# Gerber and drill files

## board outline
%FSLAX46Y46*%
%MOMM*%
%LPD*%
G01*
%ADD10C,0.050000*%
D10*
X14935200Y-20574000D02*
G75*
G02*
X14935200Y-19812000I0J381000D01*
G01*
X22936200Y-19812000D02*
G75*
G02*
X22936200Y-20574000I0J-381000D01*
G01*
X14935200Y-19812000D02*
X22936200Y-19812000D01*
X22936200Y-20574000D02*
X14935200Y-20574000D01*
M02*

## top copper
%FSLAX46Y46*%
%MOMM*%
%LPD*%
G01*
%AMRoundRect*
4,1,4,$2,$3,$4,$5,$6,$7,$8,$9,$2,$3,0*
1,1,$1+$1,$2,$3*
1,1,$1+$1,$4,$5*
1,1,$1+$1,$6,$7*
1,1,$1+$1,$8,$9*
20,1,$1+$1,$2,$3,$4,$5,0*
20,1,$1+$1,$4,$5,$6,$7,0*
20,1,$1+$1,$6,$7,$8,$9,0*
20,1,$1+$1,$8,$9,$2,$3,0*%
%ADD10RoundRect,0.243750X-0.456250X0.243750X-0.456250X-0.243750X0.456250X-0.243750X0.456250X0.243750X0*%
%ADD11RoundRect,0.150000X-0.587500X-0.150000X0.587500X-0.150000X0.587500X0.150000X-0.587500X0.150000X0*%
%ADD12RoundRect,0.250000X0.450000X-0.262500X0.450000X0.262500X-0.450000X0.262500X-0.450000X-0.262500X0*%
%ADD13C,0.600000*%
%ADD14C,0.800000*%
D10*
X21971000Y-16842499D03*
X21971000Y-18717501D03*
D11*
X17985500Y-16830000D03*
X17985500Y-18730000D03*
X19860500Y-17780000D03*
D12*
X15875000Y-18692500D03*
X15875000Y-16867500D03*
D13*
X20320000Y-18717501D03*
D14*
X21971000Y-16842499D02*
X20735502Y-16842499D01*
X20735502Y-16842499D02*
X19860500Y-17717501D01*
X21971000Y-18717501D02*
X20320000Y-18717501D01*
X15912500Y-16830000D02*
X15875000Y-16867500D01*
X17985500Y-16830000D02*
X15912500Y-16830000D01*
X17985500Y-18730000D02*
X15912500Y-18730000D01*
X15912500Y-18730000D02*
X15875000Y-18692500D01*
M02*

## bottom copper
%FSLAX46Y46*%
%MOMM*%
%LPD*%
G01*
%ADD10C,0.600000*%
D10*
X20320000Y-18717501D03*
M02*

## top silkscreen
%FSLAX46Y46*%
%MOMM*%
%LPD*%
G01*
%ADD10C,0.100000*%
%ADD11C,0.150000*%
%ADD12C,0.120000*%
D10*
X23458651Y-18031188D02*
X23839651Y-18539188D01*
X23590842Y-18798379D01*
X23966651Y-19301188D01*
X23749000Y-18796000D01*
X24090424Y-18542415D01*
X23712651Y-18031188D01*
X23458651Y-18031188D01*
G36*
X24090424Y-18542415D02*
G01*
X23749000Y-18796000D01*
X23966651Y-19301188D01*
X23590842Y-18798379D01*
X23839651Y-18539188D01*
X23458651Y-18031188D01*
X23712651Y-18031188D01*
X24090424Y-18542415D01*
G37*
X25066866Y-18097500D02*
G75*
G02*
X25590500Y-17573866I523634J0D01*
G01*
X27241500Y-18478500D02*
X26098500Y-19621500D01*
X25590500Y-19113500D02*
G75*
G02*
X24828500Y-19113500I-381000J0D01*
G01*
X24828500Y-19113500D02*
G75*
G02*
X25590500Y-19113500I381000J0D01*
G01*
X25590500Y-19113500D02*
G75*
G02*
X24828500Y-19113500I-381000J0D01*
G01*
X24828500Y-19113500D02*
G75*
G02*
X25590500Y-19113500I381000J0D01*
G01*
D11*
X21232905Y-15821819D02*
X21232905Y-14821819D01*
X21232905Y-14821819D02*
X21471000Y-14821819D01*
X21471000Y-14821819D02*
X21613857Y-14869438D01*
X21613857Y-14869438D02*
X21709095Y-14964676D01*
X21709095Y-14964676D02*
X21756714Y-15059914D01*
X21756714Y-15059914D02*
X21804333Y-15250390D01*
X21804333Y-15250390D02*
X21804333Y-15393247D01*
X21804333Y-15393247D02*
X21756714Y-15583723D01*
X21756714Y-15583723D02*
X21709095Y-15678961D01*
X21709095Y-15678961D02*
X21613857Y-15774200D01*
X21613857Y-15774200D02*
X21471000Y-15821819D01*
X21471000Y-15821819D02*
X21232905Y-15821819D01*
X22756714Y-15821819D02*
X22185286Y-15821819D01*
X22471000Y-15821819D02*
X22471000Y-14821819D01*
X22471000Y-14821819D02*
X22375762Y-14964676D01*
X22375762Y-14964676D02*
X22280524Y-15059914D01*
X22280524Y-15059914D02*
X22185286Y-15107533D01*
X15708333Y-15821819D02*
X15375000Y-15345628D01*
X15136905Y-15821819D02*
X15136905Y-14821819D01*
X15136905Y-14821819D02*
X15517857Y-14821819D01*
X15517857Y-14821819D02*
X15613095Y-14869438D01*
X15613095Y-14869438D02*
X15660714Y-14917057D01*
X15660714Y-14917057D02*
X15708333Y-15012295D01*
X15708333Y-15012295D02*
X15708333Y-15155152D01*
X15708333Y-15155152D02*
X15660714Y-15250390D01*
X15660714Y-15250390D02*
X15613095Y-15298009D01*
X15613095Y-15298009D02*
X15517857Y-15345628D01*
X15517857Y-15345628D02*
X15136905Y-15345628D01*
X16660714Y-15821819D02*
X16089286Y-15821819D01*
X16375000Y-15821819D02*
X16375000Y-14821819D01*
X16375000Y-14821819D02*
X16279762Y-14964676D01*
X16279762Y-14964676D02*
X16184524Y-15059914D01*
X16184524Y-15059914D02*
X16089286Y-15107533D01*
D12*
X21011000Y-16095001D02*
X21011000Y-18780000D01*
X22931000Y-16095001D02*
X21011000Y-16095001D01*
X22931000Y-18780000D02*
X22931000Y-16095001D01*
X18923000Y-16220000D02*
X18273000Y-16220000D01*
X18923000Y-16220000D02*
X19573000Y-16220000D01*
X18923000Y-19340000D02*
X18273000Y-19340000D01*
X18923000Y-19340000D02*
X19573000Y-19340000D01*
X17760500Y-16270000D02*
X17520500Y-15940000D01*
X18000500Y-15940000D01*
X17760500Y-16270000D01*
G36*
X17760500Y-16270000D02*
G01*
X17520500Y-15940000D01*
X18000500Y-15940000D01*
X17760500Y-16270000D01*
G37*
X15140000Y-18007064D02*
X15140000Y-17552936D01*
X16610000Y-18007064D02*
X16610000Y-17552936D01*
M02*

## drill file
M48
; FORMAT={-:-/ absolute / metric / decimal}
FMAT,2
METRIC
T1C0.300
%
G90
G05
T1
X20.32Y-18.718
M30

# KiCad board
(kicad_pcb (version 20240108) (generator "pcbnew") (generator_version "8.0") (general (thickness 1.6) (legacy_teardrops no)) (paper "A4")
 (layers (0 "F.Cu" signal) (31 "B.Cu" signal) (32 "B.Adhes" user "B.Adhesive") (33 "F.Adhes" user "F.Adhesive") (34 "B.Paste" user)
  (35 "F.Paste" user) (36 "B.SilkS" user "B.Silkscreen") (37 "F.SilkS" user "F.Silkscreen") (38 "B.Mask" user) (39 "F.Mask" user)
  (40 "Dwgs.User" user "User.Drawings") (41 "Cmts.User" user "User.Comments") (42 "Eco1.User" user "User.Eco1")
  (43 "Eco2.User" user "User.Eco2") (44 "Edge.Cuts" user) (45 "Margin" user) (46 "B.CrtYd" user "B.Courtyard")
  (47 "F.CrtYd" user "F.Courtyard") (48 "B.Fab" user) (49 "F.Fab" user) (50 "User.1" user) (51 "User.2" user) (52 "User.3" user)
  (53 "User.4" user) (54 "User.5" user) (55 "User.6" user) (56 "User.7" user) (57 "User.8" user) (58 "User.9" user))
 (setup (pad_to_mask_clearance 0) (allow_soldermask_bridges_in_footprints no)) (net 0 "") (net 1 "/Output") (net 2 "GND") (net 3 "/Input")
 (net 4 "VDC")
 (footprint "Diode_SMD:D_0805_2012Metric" (layer "F.Cu") (at 21.971 17.78 -90)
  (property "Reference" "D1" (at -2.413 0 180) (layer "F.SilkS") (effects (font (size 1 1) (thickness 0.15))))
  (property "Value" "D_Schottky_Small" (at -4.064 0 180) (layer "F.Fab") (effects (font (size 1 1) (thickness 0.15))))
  (fp_line (start -1.684999 0.96) (end 1 0.96) (stroke (width 0.12) (type solid)) (layer "F.SilkS"))
  (fp_line (start -1.684999 -0.96) (end -1.684999 0.96) (stroke (width 0.12) (type solid)) (layer "F.SilkS"))
  (fp_line (start 1 -0.96) (end -1.684999 -0.96) (stroke (width 0.12) (type solid)) (layer "F.SilkS"))
  (pad "1" smd roundrect (at -0.937501 0 270) (size 0.975 1.4) (layers "F.Cu" "F.Paste" "F.Mask") (roundrect_rratio 0.25) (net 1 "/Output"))
  (pad "2" smd roundrect (at 0.937501 0 270) (size 0.975 1.4) (layers "F.Cu" "F.Paste" "F.Mask") (roundrect_rratio 0.25) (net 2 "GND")))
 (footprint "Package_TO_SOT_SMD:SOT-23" (layer "F.Cu") (at 18.923 17.78)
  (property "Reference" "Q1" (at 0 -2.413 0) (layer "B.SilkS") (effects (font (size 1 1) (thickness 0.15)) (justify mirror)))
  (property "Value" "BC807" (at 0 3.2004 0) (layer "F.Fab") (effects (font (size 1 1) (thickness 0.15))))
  (fp_line (start 0 -1.56) (end -0.65 -1.56) (stroke (width 0.12) (type solid)) (layer "F.SilkS"))
  (fp_line (start 0 -1.56) (end 0.65 -1.56) (stroke (width 0.12) (type solid)) (layer "F.SilkS"))
  (fp_line (start 0 1.56) (end -0.65 1.56) (stroke (width 0.12) (type solid)) (layer "F.SilkS"))
  (fp_line (start 0 1.56) (end 0.65 1.56) (stroke (width 0.12) (type solid)) (layer "F.SilkS"))
  (fp_poly
   (pts (xy -1.1625 -1.51) (xy -1.4025 -1.84) (xy -0.9225 -1.84) (xy -1.1625 -1.51)) (stroke (width 0.12) (type solid)) (fill solid)
   (layer "F.SilkS"))
  (pad "1" smd roundrect (at -0.9375 -0.95) (size 1.475 0.6) (layers "F.Cu" "F.Paste" "F.Mask") (roundrect_rratio 0.25) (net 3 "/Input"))
  (pad "2" smd roundrect (at -0.9375 0.95) (size 1.475 0.6) (layers "F.Cu" "F.Paste" "F.Mask") (roundrect_rratio 0.25) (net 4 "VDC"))
  (pad "3" smd roundrect (at 0.9375 0) (size 1.475 0.6) (layers "F.Cu" "F.Paste" "F.Mask") (roundrect_rratio 0.25) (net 1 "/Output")))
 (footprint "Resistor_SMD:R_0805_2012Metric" (layer "F.Cu") (at 15.875 17.78 90)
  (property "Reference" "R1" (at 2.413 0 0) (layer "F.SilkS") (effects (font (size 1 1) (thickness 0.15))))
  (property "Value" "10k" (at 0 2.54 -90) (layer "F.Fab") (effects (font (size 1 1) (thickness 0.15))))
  (fp_line (start -0.227064 -0.735) (end 0.227064 -0.735) (stroke (width 0.12) (type solid)) (layer "F.SilkS"))
  (fp_line (start -0.227064 0.735) (end 0.227064 0.735) (stroke (width 0.12) (type solid)) (layer "F.SilkS"))
  (pad "1" smd roundrect (at -0.9125 0 90) (size 1.025 1.4) (layers "F.Cu" "F.Paste" "F.Mask") (roundrect_rratio 0.243902) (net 4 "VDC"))
  (pad "2" smd roundrect (at 0.9125 0 90) (size 1.025 1.4) (layers "F.Cu" "F.Paste" "F.Mask") (roundrect_rratio 0.243902) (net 3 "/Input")))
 (gr_poly
  (pts (xy 23.458651 18.031188) (xy 23.839651 18.539188) (xy 23.590842 18.798379) (xy 23.966651 19.301188) (xy 23.749 18.796)
   (xy 24.090424 18.542415) (xy 23.712651 18.031188))
  (stroke (width 0.1) (type solid)) (fill solid) (layer "F.SilkS"))
 (gr_arc (start 25.066866 18.0975) (mid 25.220235 17.727235) (end 25.5905 17.573866) (stroke (width 0.1) (type default)) (layer "F.SilkS"))
 (gr_line (start 27.2415 18.4785) (end 26.0985 19.6215) (stroke (width 0.1) (type default)) (layer "F.SilkS"))
 (gr_circle (center 25.2095 19.1135) (end 25.2095 18.7325) (stroke (width 0.1) (type default)) (fill none) (layer "F.SilkS"))
 (gr_circle (center 25.2095 19.1135) (end 25.2095 18.7325) (stroke (width 0.1) (type default)) (fill none) (layer "F.SilkS"))
 (gr_arc (start 14.9352 20.574) (mid 14.5542 20.193) (end 14.9352 19.812) (stroke (width 0.05) (type default)) (layer "Edge.Cuts"))
 (gr_arc (start 22.9362 19.812) (mid 23.3172 20.193) (end 22.9362 20.574) (stroke (width 0.05) (type default)) (layer "Edge.Cuts"))
 (gr_line (start 14.9352 19.812) (end 22.9362 19.812) (stroke (width 0.05) (type default)) (layer "Edge.Cuts"))
 (gr_line (start 22.9362 20.574) (end 14.9352 20.574) (stroke (width 0.05) (type default)) (layer "Edge.Cuts"))
 (segment (start 21.971 16.842499) (end 20.735502 16.842499) (width 0.8) (layer "F.Cu") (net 1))
 (segment (start 20.735502 16.842499) (end 19.8605 17.717501) (width 0.8) (layer "F.Cu") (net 1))
 (segment (start 21.971 18.717501) (end 20.32 18.717501) (width 0.8) (layer "F.Cu") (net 2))
 (via (at 20.32 18.717501) (size 0.6) (drill 0.3) (layers "F.Cu" "B.Cu") (free yes) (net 2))
 (segment (start 15.9125 16.83) (end 15.875 16.8675) (width 0.8) (layer "F.Cu") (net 3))
 (segment (start 17.9855 16.83) (end 15.9125 16.83) (width 0.8) (layer "F.Cu") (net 3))
 (segment (start 17.9855 18.73) (end 15.9125 18.73) (width 0.8) (layer "F.Cu") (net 4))
 (segment (start 15.9125 18.73) (end 15.875 18.6925) (width 0.8) (layer "F.Cu") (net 4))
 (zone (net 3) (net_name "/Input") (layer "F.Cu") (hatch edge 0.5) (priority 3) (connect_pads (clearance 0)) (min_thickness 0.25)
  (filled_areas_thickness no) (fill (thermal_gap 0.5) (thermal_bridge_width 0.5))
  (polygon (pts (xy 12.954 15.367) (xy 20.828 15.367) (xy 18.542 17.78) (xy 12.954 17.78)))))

